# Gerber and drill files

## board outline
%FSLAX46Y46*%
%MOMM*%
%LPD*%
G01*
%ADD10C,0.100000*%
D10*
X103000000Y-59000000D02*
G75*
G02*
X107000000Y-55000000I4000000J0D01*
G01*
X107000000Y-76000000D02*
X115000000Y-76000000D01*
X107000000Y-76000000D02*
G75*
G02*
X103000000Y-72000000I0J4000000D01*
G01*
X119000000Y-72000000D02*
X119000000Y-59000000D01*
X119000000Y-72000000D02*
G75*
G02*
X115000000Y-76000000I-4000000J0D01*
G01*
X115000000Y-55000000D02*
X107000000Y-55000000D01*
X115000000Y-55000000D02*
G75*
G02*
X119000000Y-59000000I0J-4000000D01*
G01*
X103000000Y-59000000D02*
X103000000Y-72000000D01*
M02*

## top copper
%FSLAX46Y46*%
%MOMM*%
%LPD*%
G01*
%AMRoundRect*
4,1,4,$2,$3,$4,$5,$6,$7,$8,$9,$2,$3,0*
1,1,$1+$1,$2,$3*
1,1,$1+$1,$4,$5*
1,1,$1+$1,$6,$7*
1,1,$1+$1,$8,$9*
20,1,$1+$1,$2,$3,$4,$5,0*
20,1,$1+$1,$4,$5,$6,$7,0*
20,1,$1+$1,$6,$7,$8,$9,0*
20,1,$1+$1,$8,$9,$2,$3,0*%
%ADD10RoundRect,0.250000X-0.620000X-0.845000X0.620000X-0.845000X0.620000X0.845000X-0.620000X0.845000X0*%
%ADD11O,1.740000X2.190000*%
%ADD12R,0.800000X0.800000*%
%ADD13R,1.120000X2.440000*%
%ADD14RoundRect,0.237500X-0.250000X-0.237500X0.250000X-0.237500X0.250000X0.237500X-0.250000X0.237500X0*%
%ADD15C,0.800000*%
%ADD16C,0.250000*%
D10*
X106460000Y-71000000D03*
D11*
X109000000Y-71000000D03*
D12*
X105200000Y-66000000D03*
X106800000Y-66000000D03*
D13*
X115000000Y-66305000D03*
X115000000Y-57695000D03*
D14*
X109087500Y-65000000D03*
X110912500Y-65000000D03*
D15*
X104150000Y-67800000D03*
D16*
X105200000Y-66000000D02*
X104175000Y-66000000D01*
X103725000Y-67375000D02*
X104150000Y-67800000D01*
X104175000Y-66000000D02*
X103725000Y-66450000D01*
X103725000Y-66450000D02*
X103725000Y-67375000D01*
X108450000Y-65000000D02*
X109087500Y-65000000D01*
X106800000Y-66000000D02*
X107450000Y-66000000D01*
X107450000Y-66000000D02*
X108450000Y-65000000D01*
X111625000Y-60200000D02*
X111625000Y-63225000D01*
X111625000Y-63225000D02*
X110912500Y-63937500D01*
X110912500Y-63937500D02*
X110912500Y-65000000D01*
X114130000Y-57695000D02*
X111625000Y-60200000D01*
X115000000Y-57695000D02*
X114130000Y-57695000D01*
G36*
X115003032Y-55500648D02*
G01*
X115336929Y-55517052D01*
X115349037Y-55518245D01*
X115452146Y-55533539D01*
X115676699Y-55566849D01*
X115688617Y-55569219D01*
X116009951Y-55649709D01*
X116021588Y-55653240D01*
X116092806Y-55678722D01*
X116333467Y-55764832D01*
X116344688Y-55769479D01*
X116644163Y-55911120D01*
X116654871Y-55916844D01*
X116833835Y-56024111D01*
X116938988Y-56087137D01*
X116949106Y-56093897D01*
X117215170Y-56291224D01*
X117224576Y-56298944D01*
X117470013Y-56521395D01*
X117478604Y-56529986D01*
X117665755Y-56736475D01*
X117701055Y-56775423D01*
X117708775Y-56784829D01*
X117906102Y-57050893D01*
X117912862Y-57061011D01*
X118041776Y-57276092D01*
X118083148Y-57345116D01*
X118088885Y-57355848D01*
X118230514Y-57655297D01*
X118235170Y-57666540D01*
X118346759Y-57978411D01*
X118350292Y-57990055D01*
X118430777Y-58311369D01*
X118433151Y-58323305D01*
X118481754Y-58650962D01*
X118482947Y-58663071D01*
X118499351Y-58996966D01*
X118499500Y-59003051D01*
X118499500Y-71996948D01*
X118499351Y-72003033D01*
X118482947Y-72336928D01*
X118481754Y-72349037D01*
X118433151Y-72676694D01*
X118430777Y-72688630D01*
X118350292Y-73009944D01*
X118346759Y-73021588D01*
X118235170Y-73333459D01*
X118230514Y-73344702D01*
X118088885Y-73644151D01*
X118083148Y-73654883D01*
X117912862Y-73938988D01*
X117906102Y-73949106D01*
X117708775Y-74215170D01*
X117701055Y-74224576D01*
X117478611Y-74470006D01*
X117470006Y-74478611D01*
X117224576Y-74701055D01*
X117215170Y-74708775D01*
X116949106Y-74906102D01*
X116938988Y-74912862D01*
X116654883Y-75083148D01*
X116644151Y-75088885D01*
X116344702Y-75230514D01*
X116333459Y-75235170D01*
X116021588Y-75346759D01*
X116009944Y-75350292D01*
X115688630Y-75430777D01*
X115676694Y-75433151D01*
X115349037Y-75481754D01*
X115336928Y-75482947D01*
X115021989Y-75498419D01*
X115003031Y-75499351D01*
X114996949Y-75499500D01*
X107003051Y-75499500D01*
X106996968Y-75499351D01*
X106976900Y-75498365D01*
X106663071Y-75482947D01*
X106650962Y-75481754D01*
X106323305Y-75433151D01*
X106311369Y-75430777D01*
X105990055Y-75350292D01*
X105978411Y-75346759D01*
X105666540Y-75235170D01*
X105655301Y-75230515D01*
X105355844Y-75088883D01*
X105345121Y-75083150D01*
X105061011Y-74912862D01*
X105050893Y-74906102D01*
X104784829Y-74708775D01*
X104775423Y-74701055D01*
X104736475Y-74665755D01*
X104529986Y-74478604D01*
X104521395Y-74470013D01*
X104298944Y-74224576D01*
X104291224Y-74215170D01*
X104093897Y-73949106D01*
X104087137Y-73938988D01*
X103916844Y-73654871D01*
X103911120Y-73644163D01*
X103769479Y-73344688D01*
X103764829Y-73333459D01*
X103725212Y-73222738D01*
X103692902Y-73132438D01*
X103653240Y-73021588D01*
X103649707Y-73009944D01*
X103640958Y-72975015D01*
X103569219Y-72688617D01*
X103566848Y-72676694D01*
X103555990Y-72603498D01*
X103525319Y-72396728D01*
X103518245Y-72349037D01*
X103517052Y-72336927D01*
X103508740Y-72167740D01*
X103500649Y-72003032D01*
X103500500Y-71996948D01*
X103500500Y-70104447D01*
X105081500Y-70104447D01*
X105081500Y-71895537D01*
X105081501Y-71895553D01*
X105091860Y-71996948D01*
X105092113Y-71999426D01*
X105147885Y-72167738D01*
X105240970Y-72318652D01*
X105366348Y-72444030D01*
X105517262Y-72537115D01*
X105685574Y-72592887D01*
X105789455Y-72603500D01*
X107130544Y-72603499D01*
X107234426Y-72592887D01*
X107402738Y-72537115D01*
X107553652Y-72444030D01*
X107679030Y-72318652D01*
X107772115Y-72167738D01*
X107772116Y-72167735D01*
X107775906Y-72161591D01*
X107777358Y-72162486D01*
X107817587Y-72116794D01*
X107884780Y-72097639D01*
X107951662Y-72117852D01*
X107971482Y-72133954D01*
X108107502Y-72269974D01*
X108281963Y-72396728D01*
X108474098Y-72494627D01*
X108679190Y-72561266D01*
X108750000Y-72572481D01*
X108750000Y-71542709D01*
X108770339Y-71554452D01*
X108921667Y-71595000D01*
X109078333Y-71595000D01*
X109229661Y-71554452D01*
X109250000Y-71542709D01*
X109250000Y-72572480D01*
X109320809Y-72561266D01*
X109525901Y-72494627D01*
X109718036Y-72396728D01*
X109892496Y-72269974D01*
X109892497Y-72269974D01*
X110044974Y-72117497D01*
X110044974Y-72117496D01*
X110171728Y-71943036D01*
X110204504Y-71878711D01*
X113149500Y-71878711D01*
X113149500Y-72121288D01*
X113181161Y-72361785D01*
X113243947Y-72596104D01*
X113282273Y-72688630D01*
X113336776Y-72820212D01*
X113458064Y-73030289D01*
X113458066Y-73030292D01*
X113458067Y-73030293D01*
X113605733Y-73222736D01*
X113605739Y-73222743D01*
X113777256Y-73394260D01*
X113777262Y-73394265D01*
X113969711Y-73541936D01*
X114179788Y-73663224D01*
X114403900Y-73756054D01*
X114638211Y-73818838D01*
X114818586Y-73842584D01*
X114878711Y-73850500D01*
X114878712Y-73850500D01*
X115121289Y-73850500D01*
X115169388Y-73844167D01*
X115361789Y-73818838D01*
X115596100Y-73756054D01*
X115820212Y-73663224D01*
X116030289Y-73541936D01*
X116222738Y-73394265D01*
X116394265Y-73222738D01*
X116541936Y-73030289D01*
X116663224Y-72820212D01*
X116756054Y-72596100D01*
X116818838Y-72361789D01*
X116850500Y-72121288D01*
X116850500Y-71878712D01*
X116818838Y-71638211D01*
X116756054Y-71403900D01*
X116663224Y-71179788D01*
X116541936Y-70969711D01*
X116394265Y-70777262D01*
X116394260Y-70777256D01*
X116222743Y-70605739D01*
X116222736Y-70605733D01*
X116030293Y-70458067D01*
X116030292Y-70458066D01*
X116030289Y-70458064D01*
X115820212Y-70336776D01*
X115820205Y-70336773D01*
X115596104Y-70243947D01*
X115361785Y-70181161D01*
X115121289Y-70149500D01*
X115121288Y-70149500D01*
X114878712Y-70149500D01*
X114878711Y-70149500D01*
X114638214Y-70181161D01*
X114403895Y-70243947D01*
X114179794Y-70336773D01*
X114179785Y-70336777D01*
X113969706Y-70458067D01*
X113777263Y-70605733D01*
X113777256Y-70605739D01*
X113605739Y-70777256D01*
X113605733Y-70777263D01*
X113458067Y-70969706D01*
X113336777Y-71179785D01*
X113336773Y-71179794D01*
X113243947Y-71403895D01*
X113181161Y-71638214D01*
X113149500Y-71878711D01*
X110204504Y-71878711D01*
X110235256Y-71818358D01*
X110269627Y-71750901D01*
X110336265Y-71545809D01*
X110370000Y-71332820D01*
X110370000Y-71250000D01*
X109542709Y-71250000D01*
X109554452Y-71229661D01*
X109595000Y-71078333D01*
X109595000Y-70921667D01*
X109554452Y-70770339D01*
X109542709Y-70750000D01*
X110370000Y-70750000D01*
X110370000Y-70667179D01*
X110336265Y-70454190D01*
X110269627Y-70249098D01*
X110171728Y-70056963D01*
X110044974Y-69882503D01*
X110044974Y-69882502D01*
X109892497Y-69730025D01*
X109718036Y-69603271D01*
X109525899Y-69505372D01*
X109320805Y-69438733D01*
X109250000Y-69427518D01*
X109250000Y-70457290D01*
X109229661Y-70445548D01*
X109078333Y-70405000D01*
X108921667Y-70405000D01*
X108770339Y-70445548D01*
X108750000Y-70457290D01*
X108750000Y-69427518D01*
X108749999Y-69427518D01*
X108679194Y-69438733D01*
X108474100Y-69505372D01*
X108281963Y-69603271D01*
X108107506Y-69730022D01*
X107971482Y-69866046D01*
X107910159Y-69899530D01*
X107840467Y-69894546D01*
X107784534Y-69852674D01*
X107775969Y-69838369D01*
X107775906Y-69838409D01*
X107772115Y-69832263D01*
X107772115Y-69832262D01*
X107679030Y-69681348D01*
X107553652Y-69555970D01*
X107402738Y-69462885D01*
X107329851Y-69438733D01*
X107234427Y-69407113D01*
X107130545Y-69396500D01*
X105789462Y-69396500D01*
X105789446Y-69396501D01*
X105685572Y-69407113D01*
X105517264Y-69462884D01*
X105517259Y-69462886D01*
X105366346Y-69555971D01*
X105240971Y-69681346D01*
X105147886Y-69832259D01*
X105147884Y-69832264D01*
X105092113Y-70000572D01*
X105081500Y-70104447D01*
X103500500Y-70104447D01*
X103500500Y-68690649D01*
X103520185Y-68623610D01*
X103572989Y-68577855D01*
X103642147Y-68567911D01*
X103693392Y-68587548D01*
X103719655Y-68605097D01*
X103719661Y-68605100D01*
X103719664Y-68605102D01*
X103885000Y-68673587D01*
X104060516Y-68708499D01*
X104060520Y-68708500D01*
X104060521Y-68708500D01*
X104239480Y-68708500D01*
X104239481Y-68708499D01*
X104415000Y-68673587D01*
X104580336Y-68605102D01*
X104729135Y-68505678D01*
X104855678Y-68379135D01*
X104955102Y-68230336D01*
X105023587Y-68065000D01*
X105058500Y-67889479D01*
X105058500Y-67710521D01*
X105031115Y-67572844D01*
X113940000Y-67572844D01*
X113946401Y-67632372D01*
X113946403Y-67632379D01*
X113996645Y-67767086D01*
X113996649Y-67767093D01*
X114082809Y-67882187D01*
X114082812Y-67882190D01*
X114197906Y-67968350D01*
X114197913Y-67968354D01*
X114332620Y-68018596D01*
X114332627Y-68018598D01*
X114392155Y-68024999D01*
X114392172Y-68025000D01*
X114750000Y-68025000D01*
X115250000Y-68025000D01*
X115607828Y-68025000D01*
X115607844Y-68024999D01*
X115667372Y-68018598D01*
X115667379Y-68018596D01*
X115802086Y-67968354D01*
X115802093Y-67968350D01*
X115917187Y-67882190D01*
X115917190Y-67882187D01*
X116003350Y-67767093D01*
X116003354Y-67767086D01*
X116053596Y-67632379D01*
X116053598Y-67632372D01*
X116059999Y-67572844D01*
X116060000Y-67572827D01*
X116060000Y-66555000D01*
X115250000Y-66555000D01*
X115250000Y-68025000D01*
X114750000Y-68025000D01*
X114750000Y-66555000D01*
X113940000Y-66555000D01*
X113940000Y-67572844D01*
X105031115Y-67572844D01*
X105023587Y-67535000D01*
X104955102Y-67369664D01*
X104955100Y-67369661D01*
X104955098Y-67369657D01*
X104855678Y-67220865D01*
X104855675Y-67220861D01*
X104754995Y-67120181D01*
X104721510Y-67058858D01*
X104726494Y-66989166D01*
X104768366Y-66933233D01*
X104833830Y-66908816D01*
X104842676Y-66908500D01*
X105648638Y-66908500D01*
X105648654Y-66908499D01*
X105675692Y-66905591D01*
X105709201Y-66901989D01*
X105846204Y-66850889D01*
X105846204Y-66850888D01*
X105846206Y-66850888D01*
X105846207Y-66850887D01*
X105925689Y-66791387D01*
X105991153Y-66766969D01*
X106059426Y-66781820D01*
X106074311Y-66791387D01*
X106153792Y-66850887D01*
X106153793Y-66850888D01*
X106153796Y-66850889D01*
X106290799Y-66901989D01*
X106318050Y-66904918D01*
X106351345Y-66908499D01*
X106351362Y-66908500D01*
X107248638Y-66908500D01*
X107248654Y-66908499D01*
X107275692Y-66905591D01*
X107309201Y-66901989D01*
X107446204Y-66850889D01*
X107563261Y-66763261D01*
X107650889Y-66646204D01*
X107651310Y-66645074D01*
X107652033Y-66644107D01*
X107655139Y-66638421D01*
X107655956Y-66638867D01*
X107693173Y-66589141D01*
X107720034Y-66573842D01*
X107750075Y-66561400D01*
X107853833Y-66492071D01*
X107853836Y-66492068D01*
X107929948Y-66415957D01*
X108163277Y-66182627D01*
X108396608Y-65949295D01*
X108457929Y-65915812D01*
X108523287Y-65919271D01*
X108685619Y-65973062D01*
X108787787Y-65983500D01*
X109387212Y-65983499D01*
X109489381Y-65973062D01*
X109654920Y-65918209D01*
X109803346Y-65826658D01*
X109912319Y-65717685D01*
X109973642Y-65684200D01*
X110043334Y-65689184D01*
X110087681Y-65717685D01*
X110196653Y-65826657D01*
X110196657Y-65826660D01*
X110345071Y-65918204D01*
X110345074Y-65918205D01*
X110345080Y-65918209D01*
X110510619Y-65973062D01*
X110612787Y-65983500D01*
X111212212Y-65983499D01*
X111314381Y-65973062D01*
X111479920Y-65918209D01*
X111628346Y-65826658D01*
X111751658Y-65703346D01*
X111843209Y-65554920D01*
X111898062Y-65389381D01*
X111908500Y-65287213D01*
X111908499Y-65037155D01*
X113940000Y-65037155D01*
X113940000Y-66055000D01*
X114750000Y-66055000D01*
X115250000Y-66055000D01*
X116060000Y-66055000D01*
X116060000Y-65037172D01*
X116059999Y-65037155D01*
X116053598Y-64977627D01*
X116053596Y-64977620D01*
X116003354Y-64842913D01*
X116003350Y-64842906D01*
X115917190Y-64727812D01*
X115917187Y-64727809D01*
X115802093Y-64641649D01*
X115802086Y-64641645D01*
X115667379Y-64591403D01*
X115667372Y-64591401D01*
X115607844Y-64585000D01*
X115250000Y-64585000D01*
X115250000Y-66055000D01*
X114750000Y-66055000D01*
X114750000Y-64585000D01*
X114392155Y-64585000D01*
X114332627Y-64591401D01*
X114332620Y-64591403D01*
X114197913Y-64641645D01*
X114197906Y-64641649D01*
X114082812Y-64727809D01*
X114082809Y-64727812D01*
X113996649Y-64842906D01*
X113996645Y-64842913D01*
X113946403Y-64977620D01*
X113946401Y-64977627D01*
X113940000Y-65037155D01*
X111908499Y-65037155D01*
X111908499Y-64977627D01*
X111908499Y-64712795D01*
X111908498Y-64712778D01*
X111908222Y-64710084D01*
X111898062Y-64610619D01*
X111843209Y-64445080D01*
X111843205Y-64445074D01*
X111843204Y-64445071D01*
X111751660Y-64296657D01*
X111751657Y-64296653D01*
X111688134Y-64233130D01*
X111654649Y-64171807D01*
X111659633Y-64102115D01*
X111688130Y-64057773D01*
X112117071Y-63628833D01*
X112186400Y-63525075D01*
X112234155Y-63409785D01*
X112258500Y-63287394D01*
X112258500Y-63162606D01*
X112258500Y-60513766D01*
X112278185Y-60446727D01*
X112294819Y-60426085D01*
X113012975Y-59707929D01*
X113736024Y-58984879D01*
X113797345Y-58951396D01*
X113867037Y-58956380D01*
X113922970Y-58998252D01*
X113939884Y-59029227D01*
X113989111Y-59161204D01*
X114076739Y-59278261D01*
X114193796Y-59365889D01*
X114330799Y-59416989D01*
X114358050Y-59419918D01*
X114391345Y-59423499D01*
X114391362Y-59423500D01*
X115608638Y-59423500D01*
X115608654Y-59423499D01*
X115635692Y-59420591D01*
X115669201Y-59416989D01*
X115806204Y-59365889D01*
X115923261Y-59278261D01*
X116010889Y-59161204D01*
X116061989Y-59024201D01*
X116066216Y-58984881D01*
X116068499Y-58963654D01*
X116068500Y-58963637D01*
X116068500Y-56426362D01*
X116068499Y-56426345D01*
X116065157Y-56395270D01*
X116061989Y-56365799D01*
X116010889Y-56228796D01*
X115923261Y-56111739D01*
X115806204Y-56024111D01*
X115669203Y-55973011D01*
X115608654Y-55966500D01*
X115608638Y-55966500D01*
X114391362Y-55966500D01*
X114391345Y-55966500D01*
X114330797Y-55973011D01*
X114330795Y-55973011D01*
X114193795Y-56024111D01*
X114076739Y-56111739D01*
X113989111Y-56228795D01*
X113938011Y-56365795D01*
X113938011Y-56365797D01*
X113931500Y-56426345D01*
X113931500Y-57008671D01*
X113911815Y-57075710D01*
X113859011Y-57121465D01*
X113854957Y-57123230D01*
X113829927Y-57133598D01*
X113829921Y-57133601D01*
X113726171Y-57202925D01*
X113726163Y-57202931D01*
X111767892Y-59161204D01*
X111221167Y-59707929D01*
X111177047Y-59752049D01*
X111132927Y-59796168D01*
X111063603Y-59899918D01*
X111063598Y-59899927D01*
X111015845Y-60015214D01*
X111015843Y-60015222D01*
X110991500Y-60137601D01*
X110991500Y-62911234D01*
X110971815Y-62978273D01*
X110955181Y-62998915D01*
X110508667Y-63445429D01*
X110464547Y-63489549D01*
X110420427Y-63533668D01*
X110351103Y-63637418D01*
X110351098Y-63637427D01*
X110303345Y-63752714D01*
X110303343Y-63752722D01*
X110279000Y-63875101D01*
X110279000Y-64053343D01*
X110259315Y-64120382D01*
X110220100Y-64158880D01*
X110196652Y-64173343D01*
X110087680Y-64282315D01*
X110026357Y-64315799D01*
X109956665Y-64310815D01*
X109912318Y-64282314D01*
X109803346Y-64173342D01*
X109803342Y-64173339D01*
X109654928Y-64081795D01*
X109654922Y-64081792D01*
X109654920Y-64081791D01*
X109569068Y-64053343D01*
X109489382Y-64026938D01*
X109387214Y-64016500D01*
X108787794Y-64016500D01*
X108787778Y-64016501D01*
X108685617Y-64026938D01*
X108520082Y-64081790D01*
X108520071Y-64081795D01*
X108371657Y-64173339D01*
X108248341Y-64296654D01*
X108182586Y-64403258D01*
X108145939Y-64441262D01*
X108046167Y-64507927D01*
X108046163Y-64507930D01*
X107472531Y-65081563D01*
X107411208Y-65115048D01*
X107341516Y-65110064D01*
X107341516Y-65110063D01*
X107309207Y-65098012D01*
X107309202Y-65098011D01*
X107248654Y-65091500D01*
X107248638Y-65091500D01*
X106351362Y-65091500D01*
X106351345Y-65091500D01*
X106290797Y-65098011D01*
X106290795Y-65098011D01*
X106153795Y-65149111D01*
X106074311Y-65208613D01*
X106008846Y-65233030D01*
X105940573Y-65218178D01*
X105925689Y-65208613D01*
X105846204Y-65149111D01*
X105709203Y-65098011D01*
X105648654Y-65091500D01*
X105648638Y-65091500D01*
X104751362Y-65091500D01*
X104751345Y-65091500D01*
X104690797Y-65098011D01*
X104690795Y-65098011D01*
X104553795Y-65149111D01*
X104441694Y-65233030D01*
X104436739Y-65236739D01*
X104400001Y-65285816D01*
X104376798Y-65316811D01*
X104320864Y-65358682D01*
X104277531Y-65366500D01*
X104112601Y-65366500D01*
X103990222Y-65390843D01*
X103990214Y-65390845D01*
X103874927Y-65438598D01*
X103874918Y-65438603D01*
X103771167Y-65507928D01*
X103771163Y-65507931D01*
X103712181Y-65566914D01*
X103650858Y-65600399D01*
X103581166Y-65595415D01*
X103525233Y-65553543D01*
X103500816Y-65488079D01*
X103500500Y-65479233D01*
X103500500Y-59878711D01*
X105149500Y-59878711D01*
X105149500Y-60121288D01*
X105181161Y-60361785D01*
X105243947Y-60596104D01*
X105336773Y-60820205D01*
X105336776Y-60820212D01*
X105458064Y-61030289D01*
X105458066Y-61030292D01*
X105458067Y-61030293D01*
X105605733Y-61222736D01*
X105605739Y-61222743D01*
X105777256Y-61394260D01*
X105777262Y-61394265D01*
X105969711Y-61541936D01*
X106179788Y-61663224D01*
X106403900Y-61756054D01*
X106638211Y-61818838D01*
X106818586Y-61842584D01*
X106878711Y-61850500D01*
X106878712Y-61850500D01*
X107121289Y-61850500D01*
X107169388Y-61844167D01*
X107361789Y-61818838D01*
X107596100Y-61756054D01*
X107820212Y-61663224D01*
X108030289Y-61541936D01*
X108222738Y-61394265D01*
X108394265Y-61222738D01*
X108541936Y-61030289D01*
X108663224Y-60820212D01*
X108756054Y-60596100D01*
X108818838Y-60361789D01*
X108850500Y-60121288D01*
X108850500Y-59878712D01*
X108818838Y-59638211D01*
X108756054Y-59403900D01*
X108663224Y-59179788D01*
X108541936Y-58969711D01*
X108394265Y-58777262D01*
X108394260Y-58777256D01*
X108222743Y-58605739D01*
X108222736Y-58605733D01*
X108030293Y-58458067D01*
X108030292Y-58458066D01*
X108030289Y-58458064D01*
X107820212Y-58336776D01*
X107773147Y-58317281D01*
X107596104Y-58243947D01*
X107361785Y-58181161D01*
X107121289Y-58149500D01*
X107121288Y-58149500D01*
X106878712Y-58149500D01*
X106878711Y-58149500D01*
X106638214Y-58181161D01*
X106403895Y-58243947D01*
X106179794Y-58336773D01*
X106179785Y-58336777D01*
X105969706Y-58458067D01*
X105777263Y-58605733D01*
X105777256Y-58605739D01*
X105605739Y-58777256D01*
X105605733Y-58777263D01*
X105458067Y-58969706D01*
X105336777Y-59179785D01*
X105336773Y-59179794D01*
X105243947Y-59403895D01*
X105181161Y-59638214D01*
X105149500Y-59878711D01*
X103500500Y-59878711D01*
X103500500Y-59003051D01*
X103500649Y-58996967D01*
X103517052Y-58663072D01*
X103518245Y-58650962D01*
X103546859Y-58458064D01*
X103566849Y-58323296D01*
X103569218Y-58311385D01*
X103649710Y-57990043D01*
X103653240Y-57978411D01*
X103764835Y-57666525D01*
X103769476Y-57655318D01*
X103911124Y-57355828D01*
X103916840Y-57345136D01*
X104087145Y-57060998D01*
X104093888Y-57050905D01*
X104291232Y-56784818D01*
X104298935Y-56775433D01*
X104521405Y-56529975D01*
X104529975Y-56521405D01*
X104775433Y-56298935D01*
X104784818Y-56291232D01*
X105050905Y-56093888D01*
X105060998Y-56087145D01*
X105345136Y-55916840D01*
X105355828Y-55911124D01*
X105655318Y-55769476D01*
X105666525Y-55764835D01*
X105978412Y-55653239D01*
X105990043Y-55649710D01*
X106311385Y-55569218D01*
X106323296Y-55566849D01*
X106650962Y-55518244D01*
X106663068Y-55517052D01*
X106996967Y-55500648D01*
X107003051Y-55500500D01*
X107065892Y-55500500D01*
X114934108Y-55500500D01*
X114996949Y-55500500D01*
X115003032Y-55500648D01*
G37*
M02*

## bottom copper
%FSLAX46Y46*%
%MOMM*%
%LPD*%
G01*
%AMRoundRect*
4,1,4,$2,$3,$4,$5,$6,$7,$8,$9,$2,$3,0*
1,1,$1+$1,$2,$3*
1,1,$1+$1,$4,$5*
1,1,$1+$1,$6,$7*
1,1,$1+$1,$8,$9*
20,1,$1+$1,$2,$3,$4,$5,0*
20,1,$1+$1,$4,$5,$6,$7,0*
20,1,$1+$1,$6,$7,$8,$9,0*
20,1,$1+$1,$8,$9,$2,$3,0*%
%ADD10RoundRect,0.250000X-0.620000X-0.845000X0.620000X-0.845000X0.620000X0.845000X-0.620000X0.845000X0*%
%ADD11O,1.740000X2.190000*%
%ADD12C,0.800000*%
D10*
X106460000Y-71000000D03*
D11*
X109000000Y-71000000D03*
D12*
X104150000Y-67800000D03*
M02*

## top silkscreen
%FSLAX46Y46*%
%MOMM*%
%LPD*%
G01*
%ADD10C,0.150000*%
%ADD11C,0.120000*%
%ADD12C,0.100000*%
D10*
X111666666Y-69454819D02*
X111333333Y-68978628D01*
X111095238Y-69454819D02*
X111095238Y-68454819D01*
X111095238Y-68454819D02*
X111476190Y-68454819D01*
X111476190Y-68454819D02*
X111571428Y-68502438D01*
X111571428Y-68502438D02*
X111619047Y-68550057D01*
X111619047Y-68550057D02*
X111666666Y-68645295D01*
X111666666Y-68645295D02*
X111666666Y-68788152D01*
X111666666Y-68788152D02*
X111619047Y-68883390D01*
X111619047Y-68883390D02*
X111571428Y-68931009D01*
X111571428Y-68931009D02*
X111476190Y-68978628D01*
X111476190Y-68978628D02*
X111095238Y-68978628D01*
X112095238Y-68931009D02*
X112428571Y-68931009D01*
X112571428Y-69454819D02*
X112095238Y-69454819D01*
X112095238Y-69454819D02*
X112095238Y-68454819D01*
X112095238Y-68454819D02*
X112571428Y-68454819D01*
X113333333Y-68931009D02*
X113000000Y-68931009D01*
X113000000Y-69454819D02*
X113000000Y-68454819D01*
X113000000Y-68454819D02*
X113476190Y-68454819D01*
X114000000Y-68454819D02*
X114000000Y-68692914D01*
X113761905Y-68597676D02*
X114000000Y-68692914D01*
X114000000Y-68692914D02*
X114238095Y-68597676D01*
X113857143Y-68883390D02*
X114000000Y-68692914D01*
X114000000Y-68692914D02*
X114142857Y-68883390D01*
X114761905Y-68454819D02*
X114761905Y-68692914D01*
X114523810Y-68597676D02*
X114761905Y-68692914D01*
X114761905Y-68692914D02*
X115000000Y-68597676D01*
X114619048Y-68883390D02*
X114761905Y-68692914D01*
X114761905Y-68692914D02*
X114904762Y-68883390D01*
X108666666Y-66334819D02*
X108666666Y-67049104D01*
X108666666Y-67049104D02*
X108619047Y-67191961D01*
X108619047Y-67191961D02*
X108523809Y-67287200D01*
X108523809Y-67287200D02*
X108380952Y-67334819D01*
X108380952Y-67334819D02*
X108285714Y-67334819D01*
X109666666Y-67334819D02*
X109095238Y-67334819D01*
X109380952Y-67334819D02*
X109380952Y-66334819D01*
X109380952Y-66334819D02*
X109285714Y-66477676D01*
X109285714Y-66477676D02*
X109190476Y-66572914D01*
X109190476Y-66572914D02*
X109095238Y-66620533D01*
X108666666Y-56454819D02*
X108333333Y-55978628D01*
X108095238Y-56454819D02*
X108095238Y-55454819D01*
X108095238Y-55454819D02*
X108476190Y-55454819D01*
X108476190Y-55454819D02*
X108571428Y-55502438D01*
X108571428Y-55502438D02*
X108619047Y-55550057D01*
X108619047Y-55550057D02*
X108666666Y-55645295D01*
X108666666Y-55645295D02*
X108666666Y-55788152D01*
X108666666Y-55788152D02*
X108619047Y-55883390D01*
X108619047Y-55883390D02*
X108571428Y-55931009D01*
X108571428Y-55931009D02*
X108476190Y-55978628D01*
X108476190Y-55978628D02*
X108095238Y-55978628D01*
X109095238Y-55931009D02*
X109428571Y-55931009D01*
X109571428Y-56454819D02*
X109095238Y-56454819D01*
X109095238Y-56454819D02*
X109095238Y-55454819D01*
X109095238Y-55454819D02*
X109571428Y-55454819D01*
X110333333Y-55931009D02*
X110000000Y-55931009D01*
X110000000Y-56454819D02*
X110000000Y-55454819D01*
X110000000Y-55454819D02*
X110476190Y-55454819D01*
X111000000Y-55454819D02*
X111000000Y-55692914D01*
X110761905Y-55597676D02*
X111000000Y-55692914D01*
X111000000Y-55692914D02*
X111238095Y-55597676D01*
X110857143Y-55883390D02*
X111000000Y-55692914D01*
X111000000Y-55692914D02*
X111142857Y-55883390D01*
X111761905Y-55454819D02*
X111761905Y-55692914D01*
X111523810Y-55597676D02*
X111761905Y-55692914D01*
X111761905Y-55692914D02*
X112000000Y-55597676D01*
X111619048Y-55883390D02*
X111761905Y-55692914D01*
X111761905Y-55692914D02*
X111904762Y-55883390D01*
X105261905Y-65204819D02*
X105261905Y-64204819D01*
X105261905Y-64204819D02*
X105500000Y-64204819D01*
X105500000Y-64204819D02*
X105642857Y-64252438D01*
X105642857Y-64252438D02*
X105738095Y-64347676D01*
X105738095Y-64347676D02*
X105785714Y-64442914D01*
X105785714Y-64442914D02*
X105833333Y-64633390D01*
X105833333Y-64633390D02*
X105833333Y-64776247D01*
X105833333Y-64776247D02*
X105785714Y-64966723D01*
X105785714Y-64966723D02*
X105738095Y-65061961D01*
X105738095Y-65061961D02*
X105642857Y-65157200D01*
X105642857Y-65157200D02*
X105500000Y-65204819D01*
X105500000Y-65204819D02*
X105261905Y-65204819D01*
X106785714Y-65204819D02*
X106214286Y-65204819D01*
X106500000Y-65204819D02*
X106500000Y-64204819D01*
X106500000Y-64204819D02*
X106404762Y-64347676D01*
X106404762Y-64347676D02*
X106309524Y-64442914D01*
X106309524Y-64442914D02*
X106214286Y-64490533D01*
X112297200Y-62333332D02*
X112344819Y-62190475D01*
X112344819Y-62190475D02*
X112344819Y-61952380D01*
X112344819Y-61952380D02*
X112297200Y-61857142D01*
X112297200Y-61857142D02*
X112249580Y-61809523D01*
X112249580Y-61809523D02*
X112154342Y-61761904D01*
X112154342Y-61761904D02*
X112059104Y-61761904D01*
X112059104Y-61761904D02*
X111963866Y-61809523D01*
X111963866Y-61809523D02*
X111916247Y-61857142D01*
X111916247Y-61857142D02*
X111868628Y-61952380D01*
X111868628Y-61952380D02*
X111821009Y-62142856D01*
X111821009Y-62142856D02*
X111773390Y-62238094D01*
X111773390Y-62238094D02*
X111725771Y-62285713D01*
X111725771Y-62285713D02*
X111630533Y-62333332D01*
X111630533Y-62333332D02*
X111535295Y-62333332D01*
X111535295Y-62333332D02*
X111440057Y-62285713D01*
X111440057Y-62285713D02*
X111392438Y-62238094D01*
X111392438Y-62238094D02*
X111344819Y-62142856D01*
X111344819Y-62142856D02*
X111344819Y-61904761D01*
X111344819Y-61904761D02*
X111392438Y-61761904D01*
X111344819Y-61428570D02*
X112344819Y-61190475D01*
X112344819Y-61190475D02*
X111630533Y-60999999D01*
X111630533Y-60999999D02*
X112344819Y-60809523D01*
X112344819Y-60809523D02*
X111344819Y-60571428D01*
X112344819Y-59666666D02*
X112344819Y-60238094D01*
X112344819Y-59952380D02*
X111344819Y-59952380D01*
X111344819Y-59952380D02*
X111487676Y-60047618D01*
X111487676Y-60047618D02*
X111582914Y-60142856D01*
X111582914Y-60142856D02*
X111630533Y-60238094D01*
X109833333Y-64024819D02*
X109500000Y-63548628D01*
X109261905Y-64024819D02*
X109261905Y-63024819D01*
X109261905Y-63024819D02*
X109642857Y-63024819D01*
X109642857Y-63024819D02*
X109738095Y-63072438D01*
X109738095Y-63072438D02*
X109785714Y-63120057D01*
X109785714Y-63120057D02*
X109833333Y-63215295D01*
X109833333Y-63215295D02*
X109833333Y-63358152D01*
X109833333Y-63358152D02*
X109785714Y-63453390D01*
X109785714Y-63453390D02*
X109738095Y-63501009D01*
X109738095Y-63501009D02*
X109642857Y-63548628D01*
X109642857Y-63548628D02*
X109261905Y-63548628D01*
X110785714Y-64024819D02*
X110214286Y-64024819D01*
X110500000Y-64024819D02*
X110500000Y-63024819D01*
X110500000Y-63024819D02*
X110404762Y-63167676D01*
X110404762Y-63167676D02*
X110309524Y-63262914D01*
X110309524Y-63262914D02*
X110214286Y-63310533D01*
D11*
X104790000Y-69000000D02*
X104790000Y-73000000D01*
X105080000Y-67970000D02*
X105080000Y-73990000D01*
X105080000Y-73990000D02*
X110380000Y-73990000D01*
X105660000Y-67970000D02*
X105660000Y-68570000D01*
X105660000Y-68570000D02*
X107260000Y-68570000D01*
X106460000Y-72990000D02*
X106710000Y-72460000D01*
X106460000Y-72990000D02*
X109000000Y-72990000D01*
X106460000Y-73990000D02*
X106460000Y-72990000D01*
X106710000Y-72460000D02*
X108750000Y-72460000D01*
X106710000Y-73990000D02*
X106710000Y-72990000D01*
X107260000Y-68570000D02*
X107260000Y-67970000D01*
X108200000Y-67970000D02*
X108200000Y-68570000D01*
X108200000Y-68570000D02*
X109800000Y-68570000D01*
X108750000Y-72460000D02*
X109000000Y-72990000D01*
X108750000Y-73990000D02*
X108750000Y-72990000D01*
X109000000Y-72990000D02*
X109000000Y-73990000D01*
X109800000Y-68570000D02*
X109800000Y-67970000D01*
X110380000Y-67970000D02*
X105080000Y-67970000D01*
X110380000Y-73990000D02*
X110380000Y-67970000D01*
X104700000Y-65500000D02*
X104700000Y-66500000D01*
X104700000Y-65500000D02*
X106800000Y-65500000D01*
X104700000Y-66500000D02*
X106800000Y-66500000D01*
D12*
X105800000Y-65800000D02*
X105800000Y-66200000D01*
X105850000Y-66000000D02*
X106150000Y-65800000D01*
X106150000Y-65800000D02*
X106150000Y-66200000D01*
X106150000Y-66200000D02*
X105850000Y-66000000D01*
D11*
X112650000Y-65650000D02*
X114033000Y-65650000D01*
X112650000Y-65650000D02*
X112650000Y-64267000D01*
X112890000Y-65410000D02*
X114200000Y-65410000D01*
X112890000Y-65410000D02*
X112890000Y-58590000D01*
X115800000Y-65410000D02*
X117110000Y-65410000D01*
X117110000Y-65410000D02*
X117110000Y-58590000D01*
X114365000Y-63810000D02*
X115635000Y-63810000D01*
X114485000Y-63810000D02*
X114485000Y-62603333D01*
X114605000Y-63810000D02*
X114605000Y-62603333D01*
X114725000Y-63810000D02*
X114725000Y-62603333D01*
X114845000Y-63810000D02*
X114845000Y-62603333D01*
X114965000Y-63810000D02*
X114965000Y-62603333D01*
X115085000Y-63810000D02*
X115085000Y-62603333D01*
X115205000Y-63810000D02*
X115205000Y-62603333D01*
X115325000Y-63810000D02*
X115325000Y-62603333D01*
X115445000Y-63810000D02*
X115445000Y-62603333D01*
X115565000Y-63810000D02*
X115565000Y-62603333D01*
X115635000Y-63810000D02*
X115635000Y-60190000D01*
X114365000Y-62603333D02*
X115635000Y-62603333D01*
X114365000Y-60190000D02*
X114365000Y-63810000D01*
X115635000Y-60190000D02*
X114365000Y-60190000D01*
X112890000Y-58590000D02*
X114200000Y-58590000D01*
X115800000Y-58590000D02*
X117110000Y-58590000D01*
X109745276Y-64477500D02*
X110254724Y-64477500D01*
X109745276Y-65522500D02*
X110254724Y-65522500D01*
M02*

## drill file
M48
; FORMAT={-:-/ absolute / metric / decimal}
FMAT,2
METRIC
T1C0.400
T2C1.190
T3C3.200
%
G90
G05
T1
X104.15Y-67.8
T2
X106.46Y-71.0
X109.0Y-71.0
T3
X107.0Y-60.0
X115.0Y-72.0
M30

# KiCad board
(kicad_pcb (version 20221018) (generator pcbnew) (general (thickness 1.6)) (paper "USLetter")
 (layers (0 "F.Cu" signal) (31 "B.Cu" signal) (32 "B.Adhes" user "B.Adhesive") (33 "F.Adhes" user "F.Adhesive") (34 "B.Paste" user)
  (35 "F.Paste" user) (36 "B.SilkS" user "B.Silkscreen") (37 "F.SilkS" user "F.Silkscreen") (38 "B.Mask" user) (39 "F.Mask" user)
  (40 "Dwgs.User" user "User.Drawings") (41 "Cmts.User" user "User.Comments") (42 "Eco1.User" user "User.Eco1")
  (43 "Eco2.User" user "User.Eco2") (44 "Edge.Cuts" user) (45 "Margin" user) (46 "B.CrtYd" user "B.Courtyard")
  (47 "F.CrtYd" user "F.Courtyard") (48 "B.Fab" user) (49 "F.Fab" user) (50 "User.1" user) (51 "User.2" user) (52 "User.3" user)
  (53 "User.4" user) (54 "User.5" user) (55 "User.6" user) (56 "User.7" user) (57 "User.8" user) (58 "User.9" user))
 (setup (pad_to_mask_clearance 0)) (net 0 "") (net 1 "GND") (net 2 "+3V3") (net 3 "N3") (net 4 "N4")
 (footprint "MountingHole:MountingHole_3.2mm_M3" (layer "F.Cu") (at 115 72)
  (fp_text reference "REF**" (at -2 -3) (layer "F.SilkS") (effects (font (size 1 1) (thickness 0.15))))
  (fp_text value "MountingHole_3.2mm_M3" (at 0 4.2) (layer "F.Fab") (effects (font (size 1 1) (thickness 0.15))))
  (pad "" np_thru_hole circle (at 0 0) (size 3.2 3.2) (drill 3.2) (layers "F&B.Cu" "*.Mask")))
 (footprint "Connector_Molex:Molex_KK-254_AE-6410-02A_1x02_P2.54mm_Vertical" (layer "F.Cu") (at 106.46 71)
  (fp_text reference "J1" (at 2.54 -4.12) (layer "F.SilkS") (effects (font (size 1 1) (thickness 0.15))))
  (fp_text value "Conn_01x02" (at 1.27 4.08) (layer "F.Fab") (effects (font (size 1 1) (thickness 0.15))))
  (fp_line (start -1.67 -2) (end -1.67 2) (stroke (width 0.12) (type solid)) (layer "F.SilkS"))
  (fp_line (start -1.38 -3.03) (end -1.38 2.99) (stroke (width 0.12) (type solid)) (layer "F.SilkS"))
  (fp_line (start -1.38 2.99) (end 3.92 2.99) (stroke (width 0.12) (type solid)) (layer "F.SilkS"))
  (fp_line (start -0.8 -3.03) (end -0.8 -2.43) (stroke (width 0.12) (type solid)) (layer "F.SilkS"))
  (fp_line (start -0.8 -2.43) (end 0.8 -2.43) (stroke (width 0.12) (type solid)) (layer "F.SilkS"))
  (fp_line (start 0 1.99) (end 0.25 1.46) (stroke (width 0.12) (type solid)) (layer "F.SilkS"))
  (fp_line (start 0 1.99) (end 2.54 1.99) (stroke (width 0.12) (type solid)) (layer "F.SilkS"))
  (fp_line (start 0 2.99) (end 0 1.99) (stroke (width 0.12) (type solid)) (layer "F.SilkS"))
  (fp_line (start 0.25 1.46) (end 2.29 1.46) (stroke (width 0.12) (type solid)) (layer "F.SilkS"))
  (fp_line (start 0.25 2.99) (end 0.25 1.99) (stroke (width 0.12) (type solid)) (layer "F.SilkS"))
  (fp_line (start 0.8 -2.43) (end 0.8 -3.03) (stroke (width 0.12) (type solid)) (layer "F.SilkS"))
  (fp_line (start 1.74 -3.03) (end 1.74 -2.43) (stroke (width 0.12) (type solid)) (layer "F.SilkS"))
  (fp_line (start 1.74 -2.43) (end 3.34 -2.43) (stroke (width 0.12) (type solid)) (layer "F.SilkS"))
  (fp_line (start 2.29 1.46) (end 2.54 1.99) (stroke (width 0.12) (type solid)) (layer "F.SilkS"))
  (fp_line (start 2.29 2.99) (end 2.29 1.99) (stroke (width 0.12) (type solid)) (layer "F.SilkS"))
  (fp_line (start 2.54 1.99) (end 2.54 2.99) (stroke (width 0.12) (type solid)) (layer "F.SilkS"))
  (fp_line (start 3.34 -2.43) (end 3.34 -3.03) (stroke (width 0.12) (type solid)) (layer "F.SilkS"))
  (fp_line (start 3.92 -3.03) (end -1.38 -3.03) (stroke (width 0.12) (type solid)) (layer "F.SilkS"))
  (fp_line (start 3.92 2.99) (end 3.92 -3.03) (stroke (width 0.12) (type solid)) (layer "F.SilkS"))
  (pad "1" thru_hole roundrect (at 0 0) (size 1.74 2.19) (drill 1.19) (layers "*.Cu" "*.Mask") (roundrect_rratio 0.143678) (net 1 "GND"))
  (pad "2" thru_hole oval (at 2.54 0) (size 1.74 2.19) (drill 1.19) (layers "*.Cu" "*.Mask") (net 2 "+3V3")))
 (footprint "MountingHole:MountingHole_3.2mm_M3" (layer "F.Cu") (at 107 60)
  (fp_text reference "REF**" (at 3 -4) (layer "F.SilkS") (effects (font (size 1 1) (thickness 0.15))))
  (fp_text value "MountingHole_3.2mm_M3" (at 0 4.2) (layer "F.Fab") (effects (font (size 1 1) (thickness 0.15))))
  (pad "" np_thru_hole circle (at 0 0) (size 3.2 3.2) (drill 3.2) (layers "*.Cu" "*.Mask")))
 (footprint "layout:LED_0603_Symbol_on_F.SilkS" (layer "F.Cu") (at 106 66)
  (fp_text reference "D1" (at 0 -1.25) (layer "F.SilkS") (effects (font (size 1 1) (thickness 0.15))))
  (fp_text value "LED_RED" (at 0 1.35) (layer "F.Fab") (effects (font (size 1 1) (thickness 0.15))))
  (fp_line (start -1.3 -0.5) (end -1.3 0.5) (stroke (width 0.12) (type solid)) (layer "F.SilkS"))
  (fp_line (start -1.3 -0.5) (end 0.8 -0.5) (stroke (width 0.12) (type solid)) (layer "F.SilkS"))
  (fp_line (start -1.3 0.5) (end 0.8 0.5) (stroke (width 0.12) (type solid)) (layer "F.SilkS"))
  (fp_line (start -0.2 -0.2) (end -0.2 0.2) (stroke (width 0.1) (type solid)) (layer "F.SilkS"))
  (fp_line (start -0.15 0) (end 0.15 -0.2) (stroke (width 0.1) (type solid)) (layer "F.SilkS"))
  (fp_line (start 0.15 -0.2) (end 0.15 0.2) (stroke (width 0.1) (type solid)) (layer "F.SilkS"))
  (fp_line (start 0.15 0.2) (end -0.15 0) (stroke (width 0.1) (type solid)) (layer "F.SilkS"))
  (pad "1" smd rect (at -0.8 0 180) (size 0.8 0.8) (layers "F.Cu" "F.Paste" "F.Mask") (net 1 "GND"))
  (pad "2" smd rect (at 0.8 0 180) (size 0.8 0.8) (layers "F.Cu" "F.Paste" "F.Mask") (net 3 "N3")))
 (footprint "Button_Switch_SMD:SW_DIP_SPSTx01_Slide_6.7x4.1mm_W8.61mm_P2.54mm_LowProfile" (layer "F.Cu") (at 115 62 90)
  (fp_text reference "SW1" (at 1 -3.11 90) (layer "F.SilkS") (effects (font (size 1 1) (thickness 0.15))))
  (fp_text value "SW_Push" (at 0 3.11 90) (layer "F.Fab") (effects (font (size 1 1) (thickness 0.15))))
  (fp_line (start -3.65 -2.35) (end -3.65 -0.967) (stroke (width 0.12) (type solid)) (layer "F.SilkS"))
  (fp_line (start -3.65 -2.35) (end -2.267 -2.35) (stroke (width 0.12) (type solid)) (layer "F.SilkS"))
  (fp_line (start -3.41 -2.11) (end -3.41 -0.8) (stroke (width 0.12) (type solid)) (layer "F.SilkS"))
  (fp_line (start -3.41 -2.11) (end 3.41 -2.11) (stroke (width 0.12) (type solid)) (layer "F.SilkS"))
  (fp_line (start -3.41 0.8) (end -3.41 2.11) (stroke (width 0.12) (type solid)) (layer "F.SilkS"))
  (fp_line (start -3.41 2.11) (end 3.41 2.11) (stroke (width 0.12) (type solid)) (layer "F.SilkS"))
  (fp_line (start -1.81 -0.635) (end -1.81 0.635) (stroke (width 0.12) (type solid)) (layer "F.SilkS"))
  (fp_line (start -1.81 -0.515) (end -0.603333 -0.515) (stroke (width 0.12) (type solid)) (layer "F.SilkS"))
  (fp_line (start -1.81 -0.395) (end -0.603333 -0.395) (stroke (width 0.12) (type solid)) (layer "F.SilkS"))
  (fp_line (start -1.81 -0.275) (end -0.603333 -0.275) (stroke (width 0.12) (type solid)) (layer "F.SilkS"))
  (fp_line (start -1.81 -0.155) (end -0.603333 -0.155) (stroke (width 0.12) (type solid)) (layer "F.SilkS"))
  (fp_line (start -1.81 -0.035) (end -0.603333 -0.035) (stroke (width 0.12) (type solid)) (layer "F.SilkS"))
  (fp_line (start -1.81 0.085) (end -0.603333 0.085) (stroke (width 0.12) (type solid)) (layer "F.SilkS"))
  (fp_line (start -1.81 0.205) (end -0.603333 0.205) (stroke (width 0.12) (type solid)) (layer "F.SilkS"))
  (fp_line (start -1.81 0.325) (end -0.603333 0.325) (stroke (width 0.12) (type solid)) (layer "F.SilkS"))
  (fp_line (start -1.81 0.445) (end -0.603333 0.445) (stroke (width 0.12) (type solid)) (layer "F.SilkS"))
  (fp_line (start -1.81 0.565) (end -0.603333 0.565) (stroke (width 0.12) (type solid)) (layer "F.SilkS"))
  (fp_line (start -1.81 0.635) (end 1.81 0.635) (stroke (width 0.12) (type solid)) (layer "F.SilkS"))
  (fp_line (start -0.603333 -0.635) (end -0.603333 0.635) (stroke (width 0.12) (type solid)) (layer "F.SilkS"))
  (fp_line (start 1.81 -0.635) (end -1.81 -0.635) (stroke (width 0.12) (type solid)) (layer "F.SilkS"))
  (fp_line (start 1.81 0.635) (end 1.81 -0.635) (stroke (width 0.12) (type solid)) (layer "F.SilkS"))
  (fp_line (start 3.41 -2.11) (end 3.41 -0.8) (stroke (width 0.12) (type solid)) (layer "F.SilkS"))
  (fp_line (start 3.41 0.8) (end 3.41 2.11) (stroke (width 0.12) (type solid)) (layer "F.SilkS"))
  (pad "1" smd rect (at -4.305 0 90) (size 2.44 1.12) (layers "F.Cu" "F.Paste" "F.Mask") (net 2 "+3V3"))
  (pad "2" smd rect (at 4.305 0 90) (size 2.44 1.12) (layers "F.Cu" "F.Paste" "F.Mask") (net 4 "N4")))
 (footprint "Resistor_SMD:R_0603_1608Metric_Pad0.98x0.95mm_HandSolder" (layer "F.Cu") (at 110 65)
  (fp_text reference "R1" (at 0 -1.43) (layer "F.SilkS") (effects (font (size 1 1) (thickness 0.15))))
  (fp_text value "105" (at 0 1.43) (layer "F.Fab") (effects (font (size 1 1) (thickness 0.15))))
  (fp_line (start -0.254724 -0.5225) (end 0.254724 -0.5225) (stroke (width 0.12) (type solid)) (layer "F.SilkS"))
  (fp_line (start -0.254724 0.5225) (end 0.254724 0.5225) (stroke (width 0.12) (type solid)) (layer "F.SilkS"))
  (pad "1" smd roundrect (at -0.9125 0) (size 0.975 0.95) (layers "F.Cu" "F.Paste" "F.Mask") (roundrect_rratio 0.25) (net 3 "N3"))
  (pad "2" smd roundrect (at 0.9125 0) (size 0.975 0.95) (layers "F.Cu" "F.Paste" "F.Mask") (roundrect_rratio 0.25) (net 4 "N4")))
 (gr_arc (start 103 59) (mid 104.171573 56.171573) (end 107 55) (stroke (width 0.1) (type default)) (layer "Edge.Cuts"))
 (gr_line (start 107 76) (end 115 76) (stroke (width 0.1) (type default)) (layer "Edge.Cuts"))
 (gr_arc (start 107 76) (mid 104.171573 74.828427) (end 103 72) (stroke (width 0.1) (type default)) (layer "Edge.Cuts"))
 (gr_line (start 119 72) (end 119 59) (stroke (width 0.1) (type default)) (layer "Edge.Cuts"))
 (gr_arc (start 119 72) (mid 117.828427 74.828427) (end 115 76) (stroke (width 0.1) (type default)) (layer "Edge.Cuts"))
 (gr_line (start 115 55) (end 107 55) (stroke (width 0.1) (type default)) (layer "Edge.Cuts"))
 (gr_arc (start 115 55) (mid 117.828427 56.171573) (end 119 59) (stroke (width 0.1) (type default)) (layer "Edge.Cuts"))
 (gr_line (start 103 59) (end 103 72) (stroke (width 0.1) (type default)) (layer "Edge.Cuts"))
 (segment (start 105.2 66) (end 104.175 66) (width 0.25) (layer "F.Cu") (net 1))
 (segment (start 103.725 67.375) (end 104.15 67.8) (width 0.25) (layer "F.Cu") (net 1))
 (segment (start 104.175 66) (end 103.725 66.45) (width 0.25) (layer "F.Cu") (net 1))
 (segment (start 103.725 66.45) (end 103.725 67.375) (width 0.25) (layer "F.Cu") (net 1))
 (via (at 104.15 67.8) (size 0.8) (drill 0.4) (layers "F.Cu" "B.Cu") (free) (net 1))
 (segment (start 108.45 65) (end 109.0875 65) (width 0.25) (layer "F.Cu") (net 3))
 (segment (start 106.8 66) (end 107.45 66) (width 0.25) (layer "F.Cu") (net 3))
 (segment (start 107.45 66) (end 108.45 65) (width 0.25) (layer "F.Cu") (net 3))
 (segment (start 111.625 60.2) (end 111.625 63.225) (width 0.25) (layer "F.Cu") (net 4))
 (segment (start 111.625 63.225) (end 110.9125 63.9375) (width 0.25) (layer "F.Cu") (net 4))
 (segment (start 110.9125 63.9375) (end 110.9125 65) (width 0.25) (layer "F.Cu") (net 4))
 (segment (start 114.13 57.695) (end 111.625 60.2) (width 0.25) (layer "F.Cu") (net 4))
 (segment (start 115 57.695) (end 114.13 57.695) (width 0.25) (layer "F.Cu") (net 4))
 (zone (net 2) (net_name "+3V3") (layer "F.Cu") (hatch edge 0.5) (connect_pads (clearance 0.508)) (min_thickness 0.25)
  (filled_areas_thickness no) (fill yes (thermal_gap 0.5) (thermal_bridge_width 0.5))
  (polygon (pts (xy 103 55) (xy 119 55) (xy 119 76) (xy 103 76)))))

